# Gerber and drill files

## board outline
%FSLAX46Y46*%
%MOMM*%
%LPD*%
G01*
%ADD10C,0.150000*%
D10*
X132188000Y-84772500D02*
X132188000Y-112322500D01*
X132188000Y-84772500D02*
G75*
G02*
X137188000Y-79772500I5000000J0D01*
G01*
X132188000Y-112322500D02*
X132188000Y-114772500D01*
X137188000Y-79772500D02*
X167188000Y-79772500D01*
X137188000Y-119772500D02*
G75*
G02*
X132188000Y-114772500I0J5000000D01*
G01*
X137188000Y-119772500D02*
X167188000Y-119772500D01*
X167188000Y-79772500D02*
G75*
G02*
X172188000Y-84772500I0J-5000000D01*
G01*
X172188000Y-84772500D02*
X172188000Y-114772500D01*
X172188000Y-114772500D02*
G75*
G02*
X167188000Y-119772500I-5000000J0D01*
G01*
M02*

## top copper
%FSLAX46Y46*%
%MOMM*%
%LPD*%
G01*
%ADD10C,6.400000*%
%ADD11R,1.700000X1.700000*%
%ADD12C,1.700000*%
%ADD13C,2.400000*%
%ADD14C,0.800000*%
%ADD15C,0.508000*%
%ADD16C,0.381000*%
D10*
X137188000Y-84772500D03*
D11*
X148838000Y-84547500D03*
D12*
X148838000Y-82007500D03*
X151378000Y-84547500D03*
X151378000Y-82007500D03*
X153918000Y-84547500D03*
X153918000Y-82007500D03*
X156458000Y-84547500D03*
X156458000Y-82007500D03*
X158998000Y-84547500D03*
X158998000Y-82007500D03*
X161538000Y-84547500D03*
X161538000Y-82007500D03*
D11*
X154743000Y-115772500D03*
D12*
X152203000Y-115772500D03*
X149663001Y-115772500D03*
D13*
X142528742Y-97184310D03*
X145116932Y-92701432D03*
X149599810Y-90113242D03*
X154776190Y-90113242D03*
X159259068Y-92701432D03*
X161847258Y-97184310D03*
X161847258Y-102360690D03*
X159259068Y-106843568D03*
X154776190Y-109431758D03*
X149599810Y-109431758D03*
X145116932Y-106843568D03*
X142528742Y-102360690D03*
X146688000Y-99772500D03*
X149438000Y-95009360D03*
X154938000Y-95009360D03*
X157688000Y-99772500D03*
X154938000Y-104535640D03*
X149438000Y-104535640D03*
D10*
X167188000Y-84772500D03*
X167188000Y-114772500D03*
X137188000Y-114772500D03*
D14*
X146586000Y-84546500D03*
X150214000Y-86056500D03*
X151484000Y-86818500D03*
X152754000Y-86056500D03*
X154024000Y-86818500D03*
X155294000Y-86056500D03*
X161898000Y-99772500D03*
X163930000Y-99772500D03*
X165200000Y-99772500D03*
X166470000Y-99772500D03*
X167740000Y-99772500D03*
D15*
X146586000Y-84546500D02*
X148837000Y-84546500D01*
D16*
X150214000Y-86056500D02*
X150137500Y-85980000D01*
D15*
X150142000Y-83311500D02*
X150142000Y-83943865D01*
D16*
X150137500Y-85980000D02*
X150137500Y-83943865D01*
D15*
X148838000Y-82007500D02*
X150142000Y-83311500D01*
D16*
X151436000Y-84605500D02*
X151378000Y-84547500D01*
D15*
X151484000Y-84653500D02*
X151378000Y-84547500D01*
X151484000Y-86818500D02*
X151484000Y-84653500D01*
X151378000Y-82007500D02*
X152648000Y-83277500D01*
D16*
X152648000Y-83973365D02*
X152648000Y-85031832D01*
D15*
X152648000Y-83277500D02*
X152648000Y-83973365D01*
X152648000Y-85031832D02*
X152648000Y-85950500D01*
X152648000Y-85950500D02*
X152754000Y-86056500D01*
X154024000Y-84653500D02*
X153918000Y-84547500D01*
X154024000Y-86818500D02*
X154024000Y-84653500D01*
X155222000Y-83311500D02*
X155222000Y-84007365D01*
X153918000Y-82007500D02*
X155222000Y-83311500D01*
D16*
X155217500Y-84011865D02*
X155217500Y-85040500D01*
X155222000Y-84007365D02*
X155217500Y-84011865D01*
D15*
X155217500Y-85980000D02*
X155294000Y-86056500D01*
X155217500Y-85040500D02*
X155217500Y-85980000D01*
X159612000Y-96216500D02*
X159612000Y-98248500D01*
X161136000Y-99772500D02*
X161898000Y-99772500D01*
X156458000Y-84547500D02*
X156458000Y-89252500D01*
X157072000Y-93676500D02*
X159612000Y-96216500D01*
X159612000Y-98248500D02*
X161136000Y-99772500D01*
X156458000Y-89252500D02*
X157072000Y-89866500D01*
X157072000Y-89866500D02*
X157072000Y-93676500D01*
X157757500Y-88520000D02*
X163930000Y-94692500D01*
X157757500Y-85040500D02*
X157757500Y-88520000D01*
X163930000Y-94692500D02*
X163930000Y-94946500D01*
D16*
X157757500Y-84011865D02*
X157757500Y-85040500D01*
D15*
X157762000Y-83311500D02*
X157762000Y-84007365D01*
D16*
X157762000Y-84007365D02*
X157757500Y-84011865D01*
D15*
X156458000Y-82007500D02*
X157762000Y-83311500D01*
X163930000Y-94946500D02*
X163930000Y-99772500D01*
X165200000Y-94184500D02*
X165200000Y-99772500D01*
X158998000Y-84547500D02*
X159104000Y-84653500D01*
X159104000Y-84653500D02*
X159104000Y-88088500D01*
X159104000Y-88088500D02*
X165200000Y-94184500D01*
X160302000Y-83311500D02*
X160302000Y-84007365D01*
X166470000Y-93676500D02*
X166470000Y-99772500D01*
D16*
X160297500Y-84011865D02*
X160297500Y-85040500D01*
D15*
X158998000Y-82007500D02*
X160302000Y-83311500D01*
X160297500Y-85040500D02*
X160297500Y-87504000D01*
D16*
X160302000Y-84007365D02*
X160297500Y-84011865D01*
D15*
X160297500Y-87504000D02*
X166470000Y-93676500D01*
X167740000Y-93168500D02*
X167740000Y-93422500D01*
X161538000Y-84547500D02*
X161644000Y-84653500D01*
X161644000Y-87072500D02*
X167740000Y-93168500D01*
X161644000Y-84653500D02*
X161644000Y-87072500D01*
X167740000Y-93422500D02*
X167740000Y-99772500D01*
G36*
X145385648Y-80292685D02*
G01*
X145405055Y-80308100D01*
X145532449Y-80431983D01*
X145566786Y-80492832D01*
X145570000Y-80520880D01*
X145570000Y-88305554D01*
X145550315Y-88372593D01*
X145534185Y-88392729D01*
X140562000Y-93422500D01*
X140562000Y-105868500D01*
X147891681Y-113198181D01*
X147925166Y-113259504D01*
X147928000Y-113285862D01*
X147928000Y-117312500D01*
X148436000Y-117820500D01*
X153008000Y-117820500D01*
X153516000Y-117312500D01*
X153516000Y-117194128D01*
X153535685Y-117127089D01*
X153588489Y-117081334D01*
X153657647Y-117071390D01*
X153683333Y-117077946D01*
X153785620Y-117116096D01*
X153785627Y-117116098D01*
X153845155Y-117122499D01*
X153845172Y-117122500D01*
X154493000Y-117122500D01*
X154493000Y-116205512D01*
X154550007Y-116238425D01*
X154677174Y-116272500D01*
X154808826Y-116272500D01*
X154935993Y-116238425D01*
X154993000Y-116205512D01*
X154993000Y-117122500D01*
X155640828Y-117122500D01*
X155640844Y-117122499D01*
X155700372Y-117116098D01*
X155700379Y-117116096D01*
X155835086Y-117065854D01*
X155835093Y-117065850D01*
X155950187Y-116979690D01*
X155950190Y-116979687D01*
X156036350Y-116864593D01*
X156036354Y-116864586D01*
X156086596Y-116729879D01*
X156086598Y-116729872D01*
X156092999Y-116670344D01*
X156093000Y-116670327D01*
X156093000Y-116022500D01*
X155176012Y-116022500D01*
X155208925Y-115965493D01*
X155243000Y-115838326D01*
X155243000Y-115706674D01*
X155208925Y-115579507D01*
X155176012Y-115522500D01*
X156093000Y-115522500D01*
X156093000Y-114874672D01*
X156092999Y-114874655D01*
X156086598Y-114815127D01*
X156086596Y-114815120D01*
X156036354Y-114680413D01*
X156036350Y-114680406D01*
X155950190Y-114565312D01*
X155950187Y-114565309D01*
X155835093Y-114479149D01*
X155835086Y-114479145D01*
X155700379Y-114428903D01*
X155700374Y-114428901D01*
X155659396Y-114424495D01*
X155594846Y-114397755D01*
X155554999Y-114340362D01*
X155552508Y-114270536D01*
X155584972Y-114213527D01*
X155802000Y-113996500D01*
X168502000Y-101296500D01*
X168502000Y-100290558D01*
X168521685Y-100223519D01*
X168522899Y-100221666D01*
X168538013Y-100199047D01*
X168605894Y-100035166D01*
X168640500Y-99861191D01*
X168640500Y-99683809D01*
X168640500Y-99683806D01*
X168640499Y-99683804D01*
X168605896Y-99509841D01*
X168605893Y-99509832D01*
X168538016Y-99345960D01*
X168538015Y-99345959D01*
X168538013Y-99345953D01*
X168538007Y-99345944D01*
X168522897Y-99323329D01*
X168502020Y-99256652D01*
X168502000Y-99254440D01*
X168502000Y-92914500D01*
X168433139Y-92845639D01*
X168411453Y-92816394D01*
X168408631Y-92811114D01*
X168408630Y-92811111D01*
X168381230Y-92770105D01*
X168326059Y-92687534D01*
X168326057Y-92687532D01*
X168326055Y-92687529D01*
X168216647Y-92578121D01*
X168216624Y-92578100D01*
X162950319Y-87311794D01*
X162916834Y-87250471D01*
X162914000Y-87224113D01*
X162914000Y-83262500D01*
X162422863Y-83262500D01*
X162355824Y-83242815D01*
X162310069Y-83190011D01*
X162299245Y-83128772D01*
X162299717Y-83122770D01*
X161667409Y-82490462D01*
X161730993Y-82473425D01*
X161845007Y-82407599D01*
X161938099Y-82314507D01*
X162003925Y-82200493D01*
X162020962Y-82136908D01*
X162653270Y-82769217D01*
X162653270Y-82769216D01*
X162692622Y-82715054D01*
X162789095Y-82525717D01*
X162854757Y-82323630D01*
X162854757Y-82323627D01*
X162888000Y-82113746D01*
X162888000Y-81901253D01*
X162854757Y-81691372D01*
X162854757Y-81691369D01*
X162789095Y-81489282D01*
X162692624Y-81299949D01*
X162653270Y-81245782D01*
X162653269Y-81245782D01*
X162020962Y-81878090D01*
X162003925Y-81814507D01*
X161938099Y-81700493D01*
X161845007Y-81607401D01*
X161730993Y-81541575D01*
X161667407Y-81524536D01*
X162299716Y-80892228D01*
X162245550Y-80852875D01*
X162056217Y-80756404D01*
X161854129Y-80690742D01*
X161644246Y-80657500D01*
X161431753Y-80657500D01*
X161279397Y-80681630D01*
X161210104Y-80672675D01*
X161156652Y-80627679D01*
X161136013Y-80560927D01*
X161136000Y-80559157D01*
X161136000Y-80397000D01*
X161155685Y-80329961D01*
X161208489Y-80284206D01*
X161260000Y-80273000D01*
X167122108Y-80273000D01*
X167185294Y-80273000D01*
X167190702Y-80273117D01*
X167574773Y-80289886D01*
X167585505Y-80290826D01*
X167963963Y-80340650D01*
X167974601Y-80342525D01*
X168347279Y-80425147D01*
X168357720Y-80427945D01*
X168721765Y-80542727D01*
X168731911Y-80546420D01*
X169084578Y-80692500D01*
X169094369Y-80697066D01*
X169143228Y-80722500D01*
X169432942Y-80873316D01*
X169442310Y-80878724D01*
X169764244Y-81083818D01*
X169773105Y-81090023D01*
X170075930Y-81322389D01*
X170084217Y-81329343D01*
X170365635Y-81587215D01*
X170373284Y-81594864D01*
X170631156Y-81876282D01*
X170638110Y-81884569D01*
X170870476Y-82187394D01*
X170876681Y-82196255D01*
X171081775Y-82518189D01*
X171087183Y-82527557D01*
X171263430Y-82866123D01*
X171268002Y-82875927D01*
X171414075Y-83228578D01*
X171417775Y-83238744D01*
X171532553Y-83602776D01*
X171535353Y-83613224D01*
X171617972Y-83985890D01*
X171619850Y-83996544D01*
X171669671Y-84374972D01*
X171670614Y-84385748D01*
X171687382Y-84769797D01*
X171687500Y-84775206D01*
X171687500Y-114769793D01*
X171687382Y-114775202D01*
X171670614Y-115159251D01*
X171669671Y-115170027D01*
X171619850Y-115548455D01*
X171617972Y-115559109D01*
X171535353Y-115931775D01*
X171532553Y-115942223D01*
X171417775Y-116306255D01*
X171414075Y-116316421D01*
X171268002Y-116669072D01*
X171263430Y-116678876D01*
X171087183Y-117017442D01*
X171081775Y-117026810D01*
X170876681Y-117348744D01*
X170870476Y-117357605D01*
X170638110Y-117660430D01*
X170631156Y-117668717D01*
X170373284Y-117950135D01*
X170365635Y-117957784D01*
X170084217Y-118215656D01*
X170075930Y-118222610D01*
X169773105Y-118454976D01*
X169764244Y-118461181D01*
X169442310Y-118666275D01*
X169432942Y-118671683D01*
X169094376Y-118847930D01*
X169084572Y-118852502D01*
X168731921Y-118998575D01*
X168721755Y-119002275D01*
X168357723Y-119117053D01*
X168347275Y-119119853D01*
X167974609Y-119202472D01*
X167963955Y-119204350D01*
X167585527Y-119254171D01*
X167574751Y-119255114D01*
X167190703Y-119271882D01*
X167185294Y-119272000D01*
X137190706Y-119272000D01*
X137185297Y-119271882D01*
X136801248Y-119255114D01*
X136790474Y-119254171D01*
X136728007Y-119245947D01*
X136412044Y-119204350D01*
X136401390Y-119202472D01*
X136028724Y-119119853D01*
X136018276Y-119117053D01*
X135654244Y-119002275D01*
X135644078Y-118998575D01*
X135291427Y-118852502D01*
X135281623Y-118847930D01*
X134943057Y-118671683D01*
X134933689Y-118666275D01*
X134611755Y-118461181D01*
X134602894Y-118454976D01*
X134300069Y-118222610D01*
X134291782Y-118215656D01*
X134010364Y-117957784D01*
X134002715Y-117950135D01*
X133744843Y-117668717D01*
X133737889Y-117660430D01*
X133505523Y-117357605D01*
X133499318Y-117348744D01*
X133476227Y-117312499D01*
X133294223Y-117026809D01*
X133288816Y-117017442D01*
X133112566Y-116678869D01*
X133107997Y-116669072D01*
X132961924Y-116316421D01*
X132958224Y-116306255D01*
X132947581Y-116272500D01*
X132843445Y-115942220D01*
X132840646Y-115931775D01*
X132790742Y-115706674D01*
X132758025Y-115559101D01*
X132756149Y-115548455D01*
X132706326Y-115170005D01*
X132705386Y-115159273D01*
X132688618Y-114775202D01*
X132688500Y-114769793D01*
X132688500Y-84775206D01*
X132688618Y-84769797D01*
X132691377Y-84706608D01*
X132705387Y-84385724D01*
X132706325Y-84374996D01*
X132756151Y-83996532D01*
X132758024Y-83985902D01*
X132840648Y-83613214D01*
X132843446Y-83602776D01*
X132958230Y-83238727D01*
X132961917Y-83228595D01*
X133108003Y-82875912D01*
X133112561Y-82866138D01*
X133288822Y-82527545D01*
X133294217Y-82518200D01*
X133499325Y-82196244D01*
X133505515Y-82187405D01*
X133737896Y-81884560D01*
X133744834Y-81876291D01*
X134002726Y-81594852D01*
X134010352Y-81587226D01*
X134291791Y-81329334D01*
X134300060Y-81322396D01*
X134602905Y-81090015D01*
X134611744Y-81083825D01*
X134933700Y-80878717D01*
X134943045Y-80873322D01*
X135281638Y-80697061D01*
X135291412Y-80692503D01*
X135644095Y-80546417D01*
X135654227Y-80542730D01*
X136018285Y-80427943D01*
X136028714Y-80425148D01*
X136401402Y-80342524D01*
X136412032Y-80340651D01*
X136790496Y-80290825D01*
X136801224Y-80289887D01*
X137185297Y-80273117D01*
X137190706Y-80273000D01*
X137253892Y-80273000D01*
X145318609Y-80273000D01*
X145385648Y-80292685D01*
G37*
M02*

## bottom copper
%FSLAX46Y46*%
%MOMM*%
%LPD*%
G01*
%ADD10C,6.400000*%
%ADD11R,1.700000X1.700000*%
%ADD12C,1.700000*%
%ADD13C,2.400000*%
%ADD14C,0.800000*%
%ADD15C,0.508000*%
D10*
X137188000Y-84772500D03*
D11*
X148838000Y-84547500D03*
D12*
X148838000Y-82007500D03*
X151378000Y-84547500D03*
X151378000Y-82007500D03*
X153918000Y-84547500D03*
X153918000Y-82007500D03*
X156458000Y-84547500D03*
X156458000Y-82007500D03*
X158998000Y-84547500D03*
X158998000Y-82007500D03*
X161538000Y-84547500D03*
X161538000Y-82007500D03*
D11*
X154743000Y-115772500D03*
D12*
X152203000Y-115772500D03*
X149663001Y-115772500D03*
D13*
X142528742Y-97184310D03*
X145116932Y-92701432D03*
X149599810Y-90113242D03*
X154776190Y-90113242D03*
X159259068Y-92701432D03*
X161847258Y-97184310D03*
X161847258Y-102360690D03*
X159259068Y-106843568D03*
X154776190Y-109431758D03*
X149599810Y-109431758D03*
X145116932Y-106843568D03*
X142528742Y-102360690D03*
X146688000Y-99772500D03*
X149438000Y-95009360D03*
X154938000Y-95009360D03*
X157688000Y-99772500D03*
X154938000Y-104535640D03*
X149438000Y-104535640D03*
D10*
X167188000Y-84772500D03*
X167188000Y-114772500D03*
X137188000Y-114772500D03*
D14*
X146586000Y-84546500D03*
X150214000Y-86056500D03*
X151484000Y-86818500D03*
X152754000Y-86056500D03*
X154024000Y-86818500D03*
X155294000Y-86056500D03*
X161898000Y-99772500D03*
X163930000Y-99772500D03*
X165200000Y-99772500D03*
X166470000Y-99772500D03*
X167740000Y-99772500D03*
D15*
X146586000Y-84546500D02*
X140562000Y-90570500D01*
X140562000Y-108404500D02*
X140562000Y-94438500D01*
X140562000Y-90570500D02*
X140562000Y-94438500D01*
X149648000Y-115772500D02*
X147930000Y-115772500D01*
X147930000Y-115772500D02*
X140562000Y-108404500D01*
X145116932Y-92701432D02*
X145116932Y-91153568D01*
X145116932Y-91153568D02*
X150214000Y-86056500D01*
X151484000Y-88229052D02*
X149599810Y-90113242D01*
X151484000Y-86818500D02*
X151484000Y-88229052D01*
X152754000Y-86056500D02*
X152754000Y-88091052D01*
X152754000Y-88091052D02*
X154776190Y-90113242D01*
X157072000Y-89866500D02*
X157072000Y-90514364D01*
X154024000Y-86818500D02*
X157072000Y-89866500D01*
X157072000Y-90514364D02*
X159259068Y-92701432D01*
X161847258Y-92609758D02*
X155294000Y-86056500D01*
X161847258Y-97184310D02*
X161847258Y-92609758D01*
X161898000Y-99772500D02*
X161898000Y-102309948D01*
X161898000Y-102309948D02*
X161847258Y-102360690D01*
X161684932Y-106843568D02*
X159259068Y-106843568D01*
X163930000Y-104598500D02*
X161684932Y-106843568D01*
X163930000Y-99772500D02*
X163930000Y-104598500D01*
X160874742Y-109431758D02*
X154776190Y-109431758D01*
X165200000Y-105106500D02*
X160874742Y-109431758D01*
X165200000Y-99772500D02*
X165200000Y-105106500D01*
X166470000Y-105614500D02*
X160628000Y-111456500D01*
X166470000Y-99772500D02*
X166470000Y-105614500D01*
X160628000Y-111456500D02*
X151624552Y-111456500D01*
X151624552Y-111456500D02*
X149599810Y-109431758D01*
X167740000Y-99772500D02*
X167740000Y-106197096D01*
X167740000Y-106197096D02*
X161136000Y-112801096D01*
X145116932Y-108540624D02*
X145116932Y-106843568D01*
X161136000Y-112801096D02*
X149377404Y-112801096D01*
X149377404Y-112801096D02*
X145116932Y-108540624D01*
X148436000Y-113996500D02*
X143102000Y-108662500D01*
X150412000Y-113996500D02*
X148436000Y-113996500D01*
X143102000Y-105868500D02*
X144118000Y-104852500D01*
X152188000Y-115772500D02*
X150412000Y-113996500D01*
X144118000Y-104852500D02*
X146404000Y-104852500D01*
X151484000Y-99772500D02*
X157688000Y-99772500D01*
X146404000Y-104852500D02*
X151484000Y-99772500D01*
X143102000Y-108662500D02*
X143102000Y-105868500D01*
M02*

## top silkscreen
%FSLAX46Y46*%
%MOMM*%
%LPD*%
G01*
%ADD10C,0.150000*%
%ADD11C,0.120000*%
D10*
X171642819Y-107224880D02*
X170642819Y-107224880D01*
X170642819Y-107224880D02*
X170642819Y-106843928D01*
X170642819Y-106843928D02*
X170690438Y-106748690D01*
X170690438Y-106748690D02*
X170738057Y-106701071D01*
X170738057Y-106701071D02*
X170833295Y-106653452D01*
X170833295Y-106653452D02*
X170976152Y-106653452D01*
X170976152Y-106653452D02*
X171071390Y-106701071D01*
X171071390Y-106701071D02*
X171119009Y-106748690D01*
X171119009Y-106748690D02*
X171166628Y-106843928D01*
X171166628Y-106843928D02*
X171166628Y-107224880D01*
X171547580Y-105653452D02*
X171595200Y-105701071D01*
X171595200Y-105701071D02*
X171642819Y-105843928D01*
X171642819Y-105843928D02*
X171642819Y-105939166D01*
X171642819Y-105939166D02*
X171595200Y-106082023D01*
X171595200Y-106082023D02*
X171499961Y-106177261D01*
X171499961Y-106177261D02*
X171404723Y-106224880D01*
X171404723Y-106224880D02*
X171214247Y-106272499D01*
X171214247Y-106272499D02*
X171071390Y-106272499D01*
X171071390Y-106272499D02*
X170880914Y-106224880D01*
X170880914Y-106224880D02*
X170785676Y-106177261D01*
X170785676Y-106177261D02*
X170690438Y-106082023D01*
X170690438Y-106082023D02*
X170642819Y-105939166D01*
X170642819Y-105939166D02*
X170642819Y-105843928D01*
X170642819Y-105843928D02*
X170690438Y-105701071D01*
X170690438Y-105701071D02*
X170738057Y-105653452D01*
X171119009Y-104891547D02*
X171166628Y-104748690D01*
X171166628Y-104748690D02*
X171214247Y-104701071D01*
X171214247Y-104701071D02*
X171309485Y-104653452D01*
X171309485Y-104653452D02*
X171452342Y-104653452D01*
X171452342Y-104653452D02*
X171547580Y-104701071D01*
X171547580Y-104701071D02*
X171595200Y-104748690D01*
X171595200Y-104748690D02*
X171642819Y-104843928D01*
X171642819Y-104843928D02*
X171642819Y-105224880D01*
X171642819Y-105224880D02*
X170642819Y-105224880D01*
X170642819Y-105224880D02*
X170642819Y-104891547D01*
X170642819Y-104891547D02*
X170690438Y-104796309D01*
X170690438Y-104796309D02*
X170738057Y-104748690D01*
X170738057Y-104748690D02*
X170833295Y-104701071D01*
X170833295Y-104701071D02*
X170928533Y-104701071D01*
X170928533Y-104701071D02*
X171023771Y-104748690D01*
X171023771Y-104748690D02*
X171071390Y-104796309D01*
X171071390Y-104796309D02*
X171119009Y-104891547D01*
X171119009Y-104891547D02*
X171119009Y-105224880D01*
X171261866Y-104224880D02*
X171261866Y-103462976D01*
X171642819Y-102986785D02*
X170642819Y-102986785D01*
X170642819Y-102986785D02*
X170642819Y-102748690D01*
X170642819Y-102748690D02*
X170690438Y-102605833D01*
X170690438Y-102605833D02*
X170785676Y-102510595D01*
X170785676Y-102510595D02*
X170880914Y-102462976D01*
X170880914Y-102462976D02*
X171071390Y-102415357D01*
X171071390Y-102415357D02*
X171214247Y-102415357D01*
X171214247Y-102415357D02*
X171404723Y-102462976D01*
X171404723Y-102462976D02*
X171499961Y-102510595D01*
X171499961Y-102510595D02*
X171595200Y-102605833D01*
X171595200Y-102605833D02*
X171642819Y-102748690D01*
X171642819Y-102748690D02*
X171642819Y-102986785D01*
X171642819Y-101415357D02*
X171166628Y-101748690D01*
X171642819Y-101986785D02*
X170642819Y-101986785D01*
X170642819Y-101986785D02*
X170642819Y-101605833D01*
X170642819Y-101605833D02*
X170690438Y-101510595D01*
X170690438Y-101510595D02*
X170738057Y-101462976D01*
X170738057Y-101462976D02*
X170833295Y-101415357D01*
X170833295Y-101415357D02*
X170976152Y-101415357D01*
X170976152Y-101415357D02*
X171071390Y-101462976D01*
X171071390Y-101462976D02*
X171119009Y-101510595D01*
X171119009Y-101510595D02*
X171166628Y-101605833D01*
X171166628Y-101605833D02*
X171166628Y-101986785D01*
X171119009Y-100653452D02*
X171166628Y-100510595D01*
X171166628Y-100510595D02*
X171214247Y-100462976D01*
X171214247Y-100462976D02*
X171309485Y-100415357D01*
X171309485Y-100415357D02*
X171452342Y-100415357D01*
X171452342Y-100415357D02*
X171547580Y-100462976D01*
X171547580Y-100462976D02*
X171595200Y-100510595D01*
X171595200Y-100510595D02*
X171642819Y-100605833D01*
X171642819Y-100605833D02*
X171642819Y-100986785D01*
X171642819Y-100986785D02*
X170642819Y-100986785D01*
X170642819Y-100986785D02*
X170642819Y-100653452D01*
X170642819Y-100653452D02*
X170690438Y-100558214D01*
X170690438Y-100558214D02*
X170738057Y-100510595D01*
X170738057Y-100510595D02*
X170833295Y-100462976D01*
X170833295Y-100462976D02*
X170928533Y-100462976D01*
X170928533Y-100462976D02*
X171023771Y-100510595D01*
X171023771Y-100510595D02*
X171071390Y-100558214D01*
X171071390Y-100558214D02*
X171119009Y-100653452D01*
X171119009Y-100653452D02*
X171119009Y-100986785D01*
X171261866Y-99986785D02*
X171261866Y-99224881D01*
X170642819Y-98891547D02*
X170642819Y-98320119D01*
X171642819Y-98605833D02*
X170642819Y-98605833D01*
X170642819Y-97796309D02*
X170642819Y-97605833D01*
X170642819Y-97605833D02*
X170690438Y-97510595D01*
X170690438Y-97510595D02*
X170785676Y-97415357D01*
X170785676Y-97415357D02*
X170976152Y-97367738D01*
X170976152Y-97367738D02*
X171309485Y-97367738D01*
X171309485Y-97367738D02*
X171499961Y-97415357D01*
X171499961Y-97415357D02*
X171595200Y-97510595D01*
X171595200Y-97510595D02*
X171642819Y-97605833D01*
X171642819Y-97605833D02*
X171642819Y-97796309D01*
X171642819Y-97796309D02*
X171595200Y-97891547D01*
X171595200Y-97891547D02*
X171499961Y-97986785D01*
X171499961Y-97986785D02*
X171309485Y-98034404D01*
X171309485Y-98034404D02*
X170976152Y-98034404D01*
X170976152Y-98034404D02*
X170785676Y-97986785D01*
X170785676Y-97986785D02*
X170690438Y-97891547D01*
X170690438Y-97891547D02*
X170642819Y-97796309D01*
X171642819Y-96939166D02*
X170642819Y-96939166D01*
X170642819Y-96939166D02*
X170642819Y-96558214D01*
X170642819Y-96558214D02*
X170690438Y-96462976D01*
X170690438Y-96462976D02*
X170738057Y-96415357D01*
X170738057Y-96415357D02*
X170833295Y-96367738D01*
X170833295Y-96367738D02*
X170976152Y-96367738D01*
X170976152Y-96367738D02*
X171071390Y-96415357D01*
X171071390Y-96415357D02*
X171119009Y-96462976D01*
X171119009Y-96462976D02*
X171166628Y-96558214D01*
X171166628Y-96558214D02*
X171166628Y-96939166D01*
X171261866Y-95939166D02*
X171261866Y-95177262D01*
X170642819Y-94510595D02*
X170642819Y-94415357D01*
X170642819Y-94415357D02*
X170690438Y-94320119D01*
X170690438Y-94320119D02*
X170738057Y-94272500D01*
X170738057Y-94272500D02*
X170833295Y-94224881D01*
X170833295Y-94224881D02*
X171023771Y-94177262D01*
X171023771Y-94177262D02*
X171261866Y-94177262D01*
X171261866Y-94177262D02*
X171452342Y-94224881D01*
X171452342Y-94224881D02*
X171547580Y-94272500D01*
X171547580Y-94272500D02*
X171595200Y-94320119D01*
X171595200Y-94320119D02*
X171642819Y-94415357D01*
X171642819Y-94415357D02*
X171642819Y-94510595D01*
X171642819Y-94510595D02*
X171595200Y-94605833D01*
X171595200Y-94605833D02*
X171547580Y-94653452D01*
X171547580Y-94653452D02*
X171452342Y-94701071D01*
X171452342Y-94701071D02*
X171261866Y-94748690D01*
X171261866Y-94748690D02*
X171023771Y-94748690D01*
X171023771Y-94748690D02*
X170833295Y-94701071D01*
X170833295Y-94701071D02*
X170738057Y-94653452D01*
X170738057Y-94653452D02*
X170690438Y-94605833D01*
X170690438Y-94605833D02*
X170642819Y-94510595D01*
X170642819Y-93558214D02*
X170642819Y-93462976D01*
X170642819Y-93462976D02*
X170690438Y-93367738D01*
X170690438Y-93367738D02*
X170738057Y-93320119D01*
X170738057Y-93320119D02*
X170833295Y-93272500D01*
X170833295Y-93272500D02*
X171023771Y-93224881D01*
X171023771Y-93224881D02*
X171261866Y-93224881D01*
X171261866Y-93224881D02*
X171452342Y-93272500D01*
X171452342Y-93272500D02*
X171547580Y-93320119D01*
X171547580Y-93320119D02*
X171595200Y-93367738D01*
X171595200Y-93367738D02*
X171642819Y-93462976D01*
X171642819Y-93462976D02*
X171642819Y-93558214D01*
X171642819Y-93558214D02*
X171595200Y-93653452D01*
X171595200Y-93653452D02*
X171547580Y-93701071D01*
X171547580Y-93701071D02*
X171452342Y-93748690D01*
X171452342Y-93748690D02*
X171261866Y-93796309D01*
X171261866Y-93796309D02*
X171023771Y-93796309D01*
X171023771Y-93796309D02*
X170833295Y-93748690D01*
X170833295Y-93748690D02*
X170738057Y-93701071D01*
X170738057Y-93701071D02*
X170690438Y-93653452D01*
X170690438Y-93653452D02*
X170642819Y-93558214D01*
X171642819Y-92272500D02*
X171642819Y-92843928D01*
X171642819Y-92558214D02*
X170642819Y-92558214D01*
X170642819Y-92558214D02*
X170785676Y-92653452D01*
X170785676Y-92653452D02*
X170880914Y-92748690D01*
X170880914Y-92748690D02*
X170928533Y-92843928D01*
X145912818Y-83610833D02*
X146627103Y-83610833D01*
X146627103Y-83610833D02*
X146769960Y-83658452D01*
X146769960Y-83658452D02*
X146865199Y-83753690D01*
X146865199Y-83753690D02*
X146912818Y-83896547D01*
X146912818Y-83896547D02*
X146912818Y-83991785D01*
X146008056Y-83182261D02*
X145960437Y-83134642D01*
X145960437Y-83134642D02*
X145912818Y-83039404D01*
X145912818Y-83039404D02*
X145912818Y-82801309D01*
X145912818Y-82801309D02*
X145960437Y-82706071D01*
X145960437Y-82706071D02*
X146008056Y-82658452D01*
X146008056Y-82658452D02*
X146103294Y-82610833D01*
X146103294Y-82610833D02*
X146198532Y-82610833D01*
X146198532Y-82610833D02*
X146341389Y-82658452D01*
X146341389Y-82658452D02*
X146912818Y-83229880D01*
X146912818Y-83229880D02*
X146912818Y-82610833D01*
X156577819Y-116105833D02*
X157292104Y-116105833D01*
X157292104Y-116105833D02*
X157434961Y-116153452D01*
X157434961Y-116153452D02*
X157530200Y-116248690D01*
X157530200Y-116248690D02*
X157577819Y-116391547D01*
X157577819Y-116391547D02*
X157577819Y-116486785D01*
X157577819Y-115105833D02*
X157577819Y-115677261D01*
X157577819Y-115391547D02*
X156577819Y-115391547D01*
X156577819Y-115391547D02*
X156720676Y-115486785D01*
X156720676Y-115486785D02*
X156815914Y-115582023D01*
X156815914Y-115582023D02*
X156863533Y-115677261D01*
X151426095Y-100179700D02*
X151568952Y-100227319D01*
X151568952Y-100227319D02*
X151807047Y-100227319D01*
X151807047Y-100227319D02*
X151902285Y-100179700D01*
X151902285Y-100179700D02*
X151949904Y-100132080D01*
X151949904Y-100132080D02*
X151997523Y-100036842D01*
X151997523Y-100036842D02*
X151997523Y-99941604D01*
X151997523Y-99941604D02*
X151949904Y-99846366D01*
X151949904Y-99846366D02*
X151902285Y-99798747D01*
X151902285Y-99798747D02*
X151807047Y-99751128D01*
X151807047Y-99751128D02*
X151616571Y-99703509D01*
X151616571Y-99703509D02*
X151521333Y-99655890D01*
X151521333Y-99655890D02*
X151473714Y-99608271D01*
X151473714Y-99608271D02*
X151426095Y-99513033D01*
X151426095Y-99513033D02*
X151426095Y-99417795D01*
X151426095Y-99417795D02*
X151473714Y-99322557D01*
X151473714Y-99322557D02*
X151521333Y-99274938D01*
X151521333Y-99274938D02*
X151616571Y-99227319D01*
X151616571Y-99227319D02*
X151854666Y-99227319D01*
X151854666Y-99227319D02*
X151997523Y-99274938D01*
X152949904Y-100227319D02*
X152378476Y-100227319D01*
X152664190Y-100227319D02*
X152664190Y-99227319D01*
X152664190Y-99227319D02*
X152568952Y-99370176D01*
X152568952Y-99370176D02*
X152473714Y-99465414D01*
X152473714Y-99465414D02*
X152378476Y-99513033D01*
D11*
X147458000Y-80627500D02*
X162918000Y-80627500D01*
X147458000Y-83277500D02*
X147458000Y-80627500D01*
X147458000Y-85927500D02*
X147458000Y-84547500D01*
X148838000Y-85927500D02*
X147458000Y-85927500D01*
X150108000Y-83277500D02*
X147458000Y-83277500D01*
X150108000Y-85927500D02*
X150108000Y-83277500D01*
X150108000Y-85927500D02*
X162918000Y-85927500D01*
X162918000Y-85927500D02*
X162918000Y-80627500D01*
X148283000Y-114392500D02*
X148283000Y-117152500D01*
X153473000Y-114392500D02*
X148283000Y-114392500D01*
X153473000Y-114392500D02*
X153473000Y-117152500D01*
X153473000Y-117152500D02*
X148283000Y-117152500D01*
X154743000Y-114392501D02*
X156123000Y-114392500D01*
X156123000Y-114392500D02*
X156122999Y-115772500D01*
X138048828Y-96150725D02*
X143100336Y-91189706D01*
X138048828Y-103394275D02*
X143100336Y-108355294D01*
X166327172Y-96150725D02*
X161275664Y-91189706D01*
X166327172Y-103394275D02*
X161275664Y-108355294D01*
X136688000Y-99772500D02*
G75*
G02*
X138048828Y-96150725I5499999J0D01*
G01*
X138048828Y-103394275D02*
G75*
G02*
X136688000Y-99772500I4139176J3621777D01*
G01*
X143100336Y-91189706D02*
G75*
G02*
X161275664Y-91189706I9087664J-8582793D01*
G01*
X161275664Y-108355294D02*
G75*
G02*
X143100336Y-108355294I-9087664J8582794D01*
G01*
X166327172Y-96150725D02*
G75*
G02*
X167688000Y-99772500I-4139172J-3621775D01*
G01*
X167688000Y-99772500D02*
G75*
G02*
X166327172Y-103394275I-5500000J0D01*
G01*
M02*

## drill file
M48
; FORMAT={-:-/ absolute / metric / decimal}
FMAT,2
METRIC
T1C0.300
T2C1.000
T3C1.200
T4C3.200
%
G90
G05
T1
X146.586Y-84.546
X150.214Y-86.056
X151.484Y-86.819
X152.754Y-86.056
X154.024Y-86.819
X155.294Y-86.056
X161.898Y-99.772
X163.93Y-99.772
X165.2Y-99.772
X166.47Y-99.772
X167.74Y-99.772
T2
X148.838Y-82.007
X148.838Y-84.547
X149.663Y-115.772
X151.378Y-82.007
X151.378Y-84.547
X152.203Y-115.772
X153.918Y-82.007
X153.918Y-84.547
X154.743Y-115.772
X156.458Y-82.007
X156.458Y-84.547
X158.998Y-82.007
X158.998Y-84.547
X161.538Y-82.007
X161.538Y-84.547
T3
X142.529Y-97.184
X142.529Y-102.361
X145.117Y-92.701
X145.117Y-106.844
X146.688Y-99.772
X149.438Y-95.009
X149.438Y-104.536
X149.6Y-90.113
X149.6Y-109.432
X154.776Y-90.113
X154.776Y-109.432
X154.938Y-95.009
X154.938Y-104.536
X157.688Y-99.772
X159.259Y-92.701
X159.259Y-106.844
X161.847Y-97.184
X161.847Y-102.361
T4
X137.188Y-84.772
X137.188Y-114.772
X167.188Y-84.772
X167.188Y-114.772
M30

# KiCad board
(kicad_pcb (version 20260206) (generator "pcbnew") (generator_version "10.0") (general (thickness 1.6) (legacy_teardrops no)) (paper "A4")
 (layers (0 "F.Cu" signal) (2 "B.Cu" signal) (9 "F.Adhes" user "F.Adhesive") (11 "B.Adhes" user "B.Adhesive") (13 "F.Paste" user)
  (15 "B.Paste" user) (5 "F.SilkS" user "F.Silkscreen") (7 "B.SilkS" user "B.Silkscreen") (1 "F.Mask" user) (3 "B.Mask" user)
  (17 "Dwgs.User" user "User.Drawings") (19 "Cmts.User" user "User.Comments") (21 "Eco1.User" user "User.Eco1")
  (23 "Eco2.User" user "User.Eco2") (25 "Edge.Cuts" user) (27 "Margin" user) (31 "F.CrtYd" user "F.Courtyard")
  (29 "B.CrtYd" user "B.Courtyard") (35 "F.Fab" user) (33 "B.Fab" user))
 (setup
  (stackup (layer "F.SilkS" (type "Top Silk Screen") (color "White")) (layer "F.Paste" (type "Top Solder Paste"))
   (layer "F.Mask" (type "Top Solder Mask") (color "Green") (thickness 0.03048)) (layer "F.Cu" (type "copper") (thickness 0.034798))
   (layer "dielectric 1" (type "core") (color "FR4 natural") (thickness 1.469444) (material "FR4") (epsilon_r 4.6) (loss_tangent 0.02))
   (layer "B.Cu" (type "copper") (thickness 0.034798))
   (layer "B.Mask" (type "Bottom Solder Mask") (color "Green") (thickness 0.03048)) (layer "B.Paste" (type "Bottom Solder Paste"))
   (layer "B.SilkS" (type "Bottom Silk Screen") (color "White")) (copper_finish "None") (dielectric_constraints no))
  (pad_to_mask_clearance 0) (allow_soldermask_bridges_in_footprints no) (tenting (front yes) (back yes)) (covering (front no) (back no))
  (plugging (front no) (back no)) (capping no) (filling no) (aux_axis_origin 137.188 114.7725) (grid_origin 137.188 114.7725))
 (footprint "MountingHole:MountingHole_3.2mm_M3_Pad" (layer "F.Cu") (at 137.188 84.7725)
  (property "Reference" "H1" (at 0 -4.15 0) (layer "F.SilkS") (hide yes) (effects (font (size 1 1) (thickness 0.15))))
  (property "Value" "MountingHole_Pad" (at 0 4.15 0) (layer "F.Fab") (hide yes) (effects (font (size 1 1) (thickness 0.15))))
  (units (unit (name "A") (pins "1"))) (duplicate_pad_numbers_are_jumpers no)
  (pad "1" thru_hole circle (at 0 0) (size 6.4 6.4) (drill 3.2) (layers "*.Cu" "*.Mask") (remove_unused_layers no) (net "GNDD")
   (zone_connect 2)))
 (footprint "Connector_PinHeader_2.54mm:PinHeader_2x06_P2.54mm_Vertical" (layer "F.Cu") (at 148.838 84.5475 90)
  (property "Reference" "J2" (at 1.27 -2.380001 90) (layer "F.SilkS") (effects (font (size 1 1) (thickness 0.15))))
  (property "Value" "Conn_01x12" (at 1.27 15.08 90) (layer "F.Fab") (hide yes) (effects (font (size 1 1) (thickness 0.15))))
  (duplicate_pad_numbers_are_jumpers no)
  (fp_line (start 3.92 -1.38) (end 3.92 14.08) (stroke (width 0.12) (type solid)) (layer "F.SilkS"))
  (fp_line (start 1.27 -1.38) (end 3.92 -1.38) (stroke (width 0.12) (type solid)) (layer "F.SilkS"))
  (fp_line (start -1.38 -1.38) (end 0 -1.38) (stroke (width 0.12) (type solid)) (layer "F.SilkS"))
  (fp_line (start -1.38 0) (end -1.38 -1.38) (stroke (width 0.12) (type solid)) (layer "F.SilkS"))
  (fp_line (start 1.27 1.27) (end 1.27 -1.38) (stroke (width 0.12) (type solid)) (layer "F.SilkS"))
  (fp_line (start -1.38 1.27) (end 1.27 1.27) (stroke (width 0.12) (type solid)) (layer "F.SilkS"))
  (fp_line (start -1.38 1.27) (end -1.38 14.08) (stroke (width 0.12) (type solid)) (layer "F.SilkS"))
  (fp_line (start -1.38 14.08) (end 3.92 14.08) (stroke (width 0.12) (type solid)) (layer "F.SilkS"))
  (pad "1" thru_hole rect (at 0 0 90) (size 1.7 1.7) (drill 1) (layers "*.Cu" "*.Mask") (remove_unused_layers no) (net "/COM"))
  (pad "2" thru_hole circle (at 2.54 0 90) (size 1.7 1.7) (drill 1) (layers "*.Cu" "*.Mask") (remove_unused_layers no) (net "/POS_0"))
  (pad "3" thru_hole circle (at 0 2.54 90) (size 1.7 1.7) (drill 1) (layers "*.Cu" "*.Mask") (remove_unused_layers no) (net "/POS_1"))
  (pad "4" thru_hole circle (at 2.54 2.54 90) (size 1.7 1.7) (drill 1) (layers "*.Cu" "*.Mask") (remove_unused_layers no) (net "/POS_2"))
  (pad "5" thru_hole circle (at 0 5.08 90) (size 1.7 1.7) (drill 1) (layers "*.Cu" "*.Mask") (remove_unused_layers no) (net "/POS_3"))
  (pad "6" thru_hole circle (at 2.54 5.08 90) (size 1.7 1.7) (drill 1) (layers "*.Cu" "*.Mask") (remove_unused_layers no) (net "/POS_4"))
  (pad "7" thru_hole circle (at 0 7.62 90) (size 1.7 1.7) (drill 1) (layers "*.Cu" "*.Mask") (remove_unused_layers no) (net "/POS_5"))
  (pad "8" thru_hole circle (at 2.54 7.62 90) (size 1.7 1.7) (drill 1) (layers "*.Cu" "*.Mask") (remove_unused_layers no) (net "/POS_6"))
  (pad "9" thru_hole circle (at 0 10.16 90) (size 1.7 1.7) (drill 1) (layers "*.Cu" "*.Mask") (remove_unused_layers no) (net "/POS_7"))
  (pad "10" thru_hole circle (at 2.54 10.16 90) (size 1.7 1.7) (drill 1) (layers "*.Cu" "*.Mask") (remove_unused_layers no) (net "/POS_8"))
  (pad "11" thru_hole circle (at 0 12.7 90) (size 1.7 1.7) (drill 1) (layers "*.Cu" "*.Mask") (remove_unused_layers no) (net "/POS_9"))
  (pad "12" thru_hole circle (at 2.54 12.7 90) (size 1.7 1.7) (drill 1) (layers "*.Cu" "*.Mask") (remove_unused_layers no) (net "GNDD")))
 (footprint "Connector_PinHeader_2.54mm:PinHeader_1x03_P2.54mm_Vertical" (layer "F.Cu") (at 154.743 115.7725 -90)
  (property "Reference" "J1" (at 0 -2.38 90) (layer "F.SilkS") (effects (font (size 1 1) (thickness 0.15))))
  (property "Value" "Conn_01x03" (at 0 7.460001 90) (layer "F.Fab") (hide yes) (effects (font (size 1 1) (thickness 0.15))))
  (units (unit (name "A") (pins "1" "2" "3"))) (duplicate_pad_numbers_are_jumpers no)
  (fp_line (start -1.38 6.46) (end 1.38 6.46) (stroke (width 0.12) (type solid)) (layer "F.SilkS"))
  (fp_line (start -1.38 1.27) (end -1.38 6.46) (stroke (width 0.12) (type solid)) (layer "F.SilkS"))
  (fp_line (start -1.38 1.27) (end 1.38 1.27) (stroke (width 0.12) (type solid)) (layer "F.SilkS"))
  (fp_line (start 1.38 1.27) (end 1.38 6.46) (stroke (width 0.12) (type solid)) (layer "F.SilkS"))
  (fp_line (start -1.379999 0) (end -1.38 -1.38) (stroke (width 0.12) (type solid)) (layer "F.SilkS"))
  (fp_line (start -1.38 -1.38) (end 0 -1.379999) (stroke (width 0.12) (type solid)) (layer "F.SilkS"))
  (pad "1" thru_hole rect (at 0 0 270) (size 1.7 1.7) (drill 1) (layers "*.Cu" "*.Mask") (remove_unused_layers no) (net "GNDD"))
  (pad "2" thru_hole circle (at 0 2.54 270) (size 1.7 1.7) (drill 1) (layers "*.Cu" "*.Mask") (remove_unused_layers no) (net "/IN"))
  (pad "3" thru_hole circle (at 0 5.079999 270) (size 1.7 1.7) (drill 1) (layers "*.Cu" "*.Mask") (remove_unused_layers no) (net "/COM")))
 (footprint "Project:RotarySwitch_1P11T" (layer "F.Cu") (at 152.188 99.7725 -90)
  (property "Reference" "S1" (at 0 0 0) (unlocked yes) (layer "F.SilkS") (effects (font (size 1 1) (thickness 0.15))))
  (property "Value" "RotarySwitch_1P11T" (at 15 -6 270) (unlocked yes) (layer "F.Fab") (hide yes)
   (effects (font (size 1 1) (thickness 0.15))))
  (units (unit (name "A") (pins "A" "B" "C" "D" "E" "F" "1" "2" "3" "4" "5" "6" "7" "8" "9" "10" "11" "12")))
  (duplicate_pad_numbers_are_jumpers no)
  (fp_line (start -3.621775 14.139172) (end -8.582794 9.087664) (stroke (width 0.12) (type default)) (layer "F.SilkS"))
  (fp_line (start 3.621775 14.139172) (end 8.582794 9.087664) (stroke (width 0.12) (type default)) (layer "F.SilkS"))
  (fp_line (start -3.621775 -14.139172) (end -8.582794 -9.087664) (stroke (width 0.12) (type default)) (layer "F.SilkS"))
  (fp_line (start 3.621775 -14.139172) (end 8.582794 -9.087664) (stroke (width 0.12) (type default)) (layer "F.SilkS"))
  (fp_arc (start 0 15.5) (mid -1.934497 15.148565) (end -3.621775 14.139172) (stroke (width 0.12) (type default)) (layer "F.SilkS"))
  (fp_arc (start 3.621775 14.139172) (mid 1.934496 15.148565) (end 0 15.5) (stroke (width 0.12) (type default)) (layer "F.SilkS"))
  (fp_arc (start -8.582794 9.087664) (mid -12.5 0) (end -8.582794 -9.087664) (stroke (width 0.12) (type default)) (layer "F.SilkS"))
  (fp_arc (start 8.582794 -9.087664) (mid 12.5 0) (end 8.582794 9.087664) (stroke (width 0.12) (type default)) (layer "F.SilkS"))
  (fp_arc (start -3.621775 -14.139172) (mid -1.934496 -15.148565) (end 0 -15.5) (stroke (width 0.12) (type default)) (layer "F.SilkS"))
  (fp_arc (start 0 -15.5) (mid 1.934497 -15.148565) (end 3.621775 -14.139172) (stroke (width 0.12) (type default)) (layer "F.SilkS"))
  (pad "1" thru_hole circle (at -2.58819 9.659258 270) (size 2.4 2.4) (drill 1.2) (layers "*.Cu" "*.Mask") (remove_unused_layers no)
   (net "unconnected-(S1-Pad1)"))
  (pad "2" thru_hole circle (at -7.071068 7.071068 270) (size 2.4 2.4) (drill 1.2) (layers "*.Cu" "*.Mask") (remove_unused_layers no)
   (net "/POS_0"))
  (pad "3" thru_hole circle (at -9.659258 2.58819 270) (size 2.4 2.4) (drill 1.2) (layers "*.Cu" "*.Mask") (remove_unused_layers no)
   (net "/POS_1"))
  (pad "4" thru_hole circle (at -9.659258 -2.58819 270) (size 2.4 2.4) (drill 1.2) (layers "*.Cu" "*.Mask") (remove_unused_layers no)
   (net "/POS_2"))
  (pad "5" thru_hole circle (at -7.071068 -7.071068 270) (size 2.4 2.4) (drill 1.2) (layers "*.Cu" "*.Mask") (remove_unused_layers no)
   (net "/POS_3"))
  (pad "6" thru_hole circle (at -2.58819 -9.659258 270) (size 2.4 2.4) (drill 1.2) (layers "*.Cu" "*.Mask") (remove_unused_layers no)
   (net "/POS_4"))
  (pad "7" thru_hole circle (at 2.58819 -9.659258 270) (size 2.4 2.4) (drill 1.2) (layers "*.Cu" "*.Mask") (remove_unused_layers no)
   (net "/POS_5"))
  (pad "8" thru_hole circle (at 7.071068 -7.071068 270) (size 2.4 2.4) (drill 1.2) (layers "*.Cu" "*.Mask") (remove_unused_layers no)
   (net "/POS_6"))
  (pad "9" thru_hole circle (at 9.659258 -2.58819 270) (size 2.4 2.4) (drill 1.2) (layers "*.Cu" "*.Mask") (remove_unused_layers no)
   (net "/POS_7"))
  (pad "10" thru_hole circle (at 9.659258 2.58819 270) (size 2.4 2.4) (drill 1.2) (layers "*.Cu" "*.Mask") (remove_unused_layers no)
   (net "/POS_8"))
  (pad "11" thru_hole circle (at 7.071068 7.071068 270) (size 2.4 2.4) (drill 1.2) (layers "*.Cu" "*.Mask") (remove_unused_layers no)
   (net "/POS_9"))
  (pad "12" thru_hole circle (at 2.58819 9.659258 270) (size 2.4 2.4) (drill 1.2) (layers "*.Cu" "*.Mask") (remove_unused_layers no)
   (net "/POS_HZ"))
  (pad "A" thru_hole circle (at 0 5.5 270) (size 2.4 2.4) (drill 1.2) (layers "*.Cu" "*.Mask") (remove_unused_layers no)
   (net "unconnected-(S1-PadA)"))
  (pad "B" thru_hole circle (at -4.76314 2.75 270) (size 2.4 2.4) (drill 1.2) (layers "*.Cu" "*.Mask") (remove_unused_layers no)
   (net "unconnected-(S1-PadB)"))
  (pad "C" thru_hole circle (at -4.76314 -2.75 270) (size 2.4 2.4) (drill 1.2) (layers "*.Cu" "*.Mask") (remove_unused_layers no)
   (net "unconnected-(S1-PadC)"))
  (pad "D" thru_hole circle (at 0 -5.5 270) (size 2.4 2.4) (drill 1.2) (layers "*.Cu" "*.Mask") (remove_unused_layers no) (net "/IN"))
  (pad "E" thru_hole circle (at 4.76314 -2.75 270) (size 2.4 2.4) (drill 1.2) (layers "*.Cu" "*.Mask") (remove_unused_layers no)
   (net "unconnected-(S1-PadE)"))
  (pad "F" thru_hole circle (at 4.76314 2.75 270) (size 2.4 2.4) (drill 1.2) (layers "*.Cu" "*.Mask") (remove_unused_layers no)
   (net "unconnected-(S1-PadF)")))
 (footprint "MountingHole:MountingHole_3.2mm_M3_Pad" (layer "F.Cu") (at 167.188 84.7725)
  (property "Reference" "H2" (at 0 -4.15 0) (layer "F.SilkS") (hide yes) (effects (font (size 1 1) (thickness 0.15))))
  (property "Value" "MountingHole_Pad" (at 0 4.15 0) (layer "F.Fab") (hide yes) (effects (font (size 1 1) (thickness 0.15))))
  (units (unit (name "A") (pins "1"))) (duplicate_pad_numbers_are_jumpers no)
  (pad "1" thru_hole circle (at 0 0) (size 6.4 6.4) (drill 3.2) (layers "*.Cu" "*.Mask") (remove_unused_layers no) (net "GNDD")
   (zone_connect 2)))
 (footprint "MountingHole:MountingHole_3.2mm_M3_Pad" (layer "F.Cu") (at 167.188 114.7725)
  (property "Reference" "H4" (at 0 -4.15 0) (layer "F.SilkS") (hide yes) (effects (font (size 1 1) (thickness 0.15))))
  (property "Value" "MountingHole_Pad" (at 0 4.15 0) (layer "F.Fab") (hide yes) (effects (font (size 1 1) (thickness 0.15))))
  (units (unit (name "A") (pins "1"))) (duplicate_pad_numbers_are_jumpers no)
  (pad "1" thru_hole circle (at 0 0) (size 6.4 6.4) (drill 3.2) (layers "*.Cu" "*.Mask") (remove_unused_layers no) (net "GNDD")
   (zone_connect 2)))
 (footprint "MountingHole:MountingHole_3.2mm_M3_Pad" (layer "F.Cu") (at 137.188 114.7725)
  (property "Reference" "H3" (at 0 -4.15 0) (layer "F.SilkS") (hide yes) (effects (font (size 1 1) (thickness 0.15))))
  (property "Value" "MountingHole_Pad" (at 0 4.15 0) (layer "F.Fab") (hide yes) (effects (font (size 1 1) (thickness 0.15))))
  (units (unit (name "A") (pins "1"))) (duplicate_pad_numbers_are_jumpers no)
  (pad "1" thru_hole circle (at 0 0) (size 6.4 6.4) (drill 3.2) (layers "*.Cu" "*.Mask") (remove_unused_layers no) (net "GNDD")
   (zone_connect 2)))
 (gr_line (start 132.188 84.7725) (end 132.188 112.3225) (stroke (width 0.15) (type default)) (layer "Edge.Cuts"))
 (gr_arc (start 132.188 84.7725) (mid 133.652466 81.236966) (end 137.188 79.7725) (stroke (width 0.15) (type default)) (layer "Edge.Cuts"))
 (gr_line (start 132.188 112.3225) (end 132.188 114.7725) (stroke (width 0.15) (type default)) (layer "Edge.Cuts"))
 (gr_line (start 137.188 79.7725) (end 167.188 79.7725) (stroke (width 0.15) (type default)) (layer "Edge.Cuts"))
 (gr_arc (start 137.188 119.7725) (mid 133.652466 118.308034) (end 132.188 114.7725) (stroke (width 0.15) (type default))
  (layer "Edge.Cuts"))
 (gr_line (start 137.188 119.7725) (end 167.188 119.7725) (stroke (width 0.15) (type default)) (layer "Edge.Cuts"))
 (gr_arc (start 167.188 79.7725) (mid 170.723534 81.236966) (end 172.188 84.7725) (stroke (width 0.15) (type default)) (layer "Edge.Cuts"))
 (gr_line (start 172.188 84.7725) (end 172.188 114.7725) (stroke (width 0.15) (type default)) (layer "Edge.Cuts"))
 (gr_arc (start 172.188 114.7725) (mid 170.723534 118.308034) (end 167.188 119.7725) (stroke (width 0.15) (type default))
  (layer "Edge.Cuts"))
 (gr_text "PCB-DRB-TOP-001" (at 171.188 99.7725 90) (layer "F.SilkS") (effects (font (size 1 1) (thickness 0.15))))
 (segment (start 146.586 84.5465) (end 148.837 84.5465) (width 0.508) (layer "F.Cu") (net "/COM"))
 (via (at 146.586 84.5465) (size 0.8) (drill 0.3) (layers "F.Cu" "B.Cu") (capping no) (covering (front no) (back no))
  (plugging (front no) (back no)) (filling no) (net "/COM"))
 (segment (start 146.586 84.5465) (end 140.562 90.5705) (width 0.508) (layer "B.Cu") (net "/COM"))
 (segment (start 140.562 108.4045) (end 140.562 94.4385) (width 0.508) (layer "B.Cu") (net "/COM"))
 (segment (start 140.562 90.5705) (end 140.562 94.4385) (width 0.508) (layer "B.Cu") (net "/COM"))
 (segment (start 149.648 115.7725) (end 147.93 115.7725) (width 0.508) (layer "B.Cu") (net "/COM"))
 (segment (start 147.93 115.7725) (end 140.562 108.4045) (width 0.508) (layer "B.Cu") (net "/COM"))
 (segment (start 150.214 86.0565) (end 150.1375 85.98) (width 0.381) (layer "F.Cu") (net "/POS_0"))
 (segment (start 150.142 83.3115) (end 150.142 83.943865) (width 0.508) (layer "F.Cu") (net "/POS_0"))
 (segment (start 150.1375 85.98) (end 150.1375 83.943865) (width 0.381) (layer "F.Cu") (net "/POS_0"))
 (segment (start 148.838 82.0075) (end 150.142 83.3115) (width 0.508) (layer "F.Cu") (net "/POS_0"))
 (via (at 150.214 86.0565) (size 0.8) (drill 0.3) (layers "F.Cu" "B.Cu") (capping no) (covering (front no) (back no))
  (plugging (front no) (back no)) (filling no) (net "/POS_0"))
 (segment (start 145.116932 92.701432) (end 145.116932 91.153568) (width 0.508) (layer "B.Cu") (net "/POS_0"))
 (segment (start 145.116932 91.153568) (end 150.214 86.0565) (width 0.508) (layer "B.Cu") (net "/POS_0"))
 (segment (start 151.436 84.6055) (end 151.378 84.5475) (width 0.381) (layer "F.Cu") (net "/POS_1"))
 (segment (start 151.484 84.6535) (end 151.378 84.5475) (width 0.508) (layer "F.Cu") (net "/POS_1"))
 (segment (start 151.484 86.8185) (end 151.484 84.6535) (width 0.508) (layer "F.Cu") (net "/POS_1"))
 (via (at 151.484 86.8185) (size 0.8) (drill 0.3) (layers "F.Cu" "B.Cu") (capping no) (covering (front no) (back no))
  (plugging (front no) (back no)) (filling no) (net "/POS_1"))
 (segment (start 151.484 88.229052) (end 149.59981 90.113242) (width 0.508) (layer "B.Cu") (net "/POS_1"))
 (segment (start 151.484 86.8185) (end 151.484 88.229052) (width 0.508) (layer "B.Cu") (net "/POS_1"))
 (segment (start 151.378 82.0075) (end 152.648 83.2775) (width 0.508) (layer "F.Cu") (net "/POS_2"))
 (segment (start 152.648 83.973365) (end 152.648 85.031832) (width 0.381) (layer "F.Cu") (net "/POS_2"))
 (segment (start 152.648 83.2775) (end 152.648 83.973365) (width 0.508) (layer "F.Cu") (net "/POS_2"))
 (segment (start 152.648 85.031832) (end 152.648 85.9505) (width 0.508) (layer "F.Cu") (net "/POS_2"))
 (segment (start 152.648 85.9505) (end 152.754 86.0565) (width 0.508) (layer "F.Cu") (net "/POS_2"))
 (via (at 152.754 86.0565) (size 0.8) (drill 0.3) (layers "F.Cu" "B.Cu") (capping no) (covering (front no) (back no))
  (plugging (front no) (back no)) (filling no) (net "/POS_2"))
 (segment (start 152.754 86.0565) (end 152.754 88.091052) (width 0.508) (layer "B.Cu") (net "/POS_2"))
 (segment (start 152.754 88.091052) (end 154.77619 90.113242) (width 0.508) (layer "B.Cu") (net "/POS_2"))
 (segment (start 154.024 84.6535) (end 153.918 84.5475) (width 0.508) (layer "F.Cu") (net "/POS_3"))
 (segment (start 154.024 86.8185) (end 154.024 84.6535) (width 0.508) (layer "F.Cu") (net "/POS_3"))
 (via (at 154.024 86.8185) (size 0.8) (drill 0.3) (layers "F.Cu" "B.Cu") (capping no) (covering (front no) (back no))
  (plugging (front no) (back no)) (filling no) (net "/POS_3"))
 (segment (start 157.072 89.8665) (end 157.072 90.514364) (width 0.508) (layer "B.Cu") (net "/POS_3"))
 (segment (start 154.024 86.8185) (end 157.072 89.8665) (width 0.508) (layer "B.Cu") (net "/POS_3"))
 (segment (start 157.072 90.514364) (end 159.259068 92.701432) (width 0.508) (layer "B.Cu") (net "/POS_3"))
 (segment (start 155.222 83.3115) (end 155.222 84.007365) (width 0.508) (layer "F.Cu") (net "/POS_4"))
 (segment (start 153.918 82.0075) (end 155.222 83.3115) (width 0.508) (layer "F.Cu") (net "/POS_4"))
 (segment (start 155.2175 84.011865) (end 155.2175 85.0405) (width 0.381) (layer "F.Cu") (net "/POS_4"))
 (segment (start 155.222 84.007365) (end 155.2175 84.011865) (width 0.381) (layer "F.Cu") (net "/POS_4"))
 (segment (start 155.2175 85.98) (end 155.294 86.0565) (width 0.508) (layer "F.Cu") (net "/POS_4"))
 (segment (start 155.2175 85.0405) (end 155.2175 85.98) (width 0.508) (layer "F.Cu") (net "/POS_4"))
 (via (at 155.294 86.0565) (size 0.8) (drill 0.3) (layers "F.Cu" "B.Cu") (capping no) (covering (front no) (back no))
  (plugging (front no) (back no)) (filling no) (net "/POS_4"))
 (segment (start 161.847258 92.609758) (end 155.294 86.0565) (width 0.508) (layer "B.Cu") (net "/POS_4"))
 (segment (start 161.847258 97.18431) (end 161.847258 92.609758) (width 0.508) (layer "B.Cu") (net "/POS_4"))
 (segment (start 159.612 96.2165) (end 159.612 98.2485) (width 0.508) (layer "F.Cu") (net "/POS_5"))
 (segment (start 161.136 99.7725) (end 161.898 99.7725) (width 0.508) (layer "F.Cu") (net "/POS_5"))
 (segment (start 156.458 84.5475) (end 156.458 89.2525) (width 0.508) (layer "F.Cu") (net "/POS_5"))
 (segment (start 157.072 93.6765) (end 159.612 96.2165) (width 0.508) (layer "F.Cu") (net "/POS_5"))
 (segment (start 159.612 98.2485) (end 161.136 99.7725) (width 0.508) (layer "F.Cu") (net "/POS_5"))
 (segment (start 156.458 89.2525) (end 157.072 89.8665) (width 0.508) (layer "F.Cu") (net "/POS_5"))
 (segment (start 157.072 89.8665) (end 157.072 93.6765) (width 0.508) (layer "F.Cu") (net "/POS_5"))
 (via (at 161.898 99.7725) (size 0.8) (drill 0.3) (layers "F.Cu" "B.Cu") (capping no) (covering (front no) (back no))
  (plugging (front no) (back no)) (filling no) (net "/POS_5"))
 (segment (start 161.898 99.7725) (end 161.898 102.309948) (width 0.508) (layer "B.Cu") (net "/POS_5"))
 (segment (start 161.898 102.309948) (end 161.847258 102.36069) (width 0.508) (layer "B.Cu") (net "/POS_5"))
 (segment (start 157.7575 88.52) (end 163.93 94.6925) (width 0.508) (layer "F.Cu") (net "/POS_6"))
 (segment (start 157.7575 85.0405) (end 157.7575 88.52) (width 0.508) (layer "F.Cu") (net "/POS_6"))
 (segment (start 163.93 94.6925) (end 163.93 94.9465) (width 0.508) (layer "F.Cu") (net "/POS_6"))
 (segment (start 157.7575 84.011865) (end 157.7575 85.0405) (width 0.381) (layer "F.Cu") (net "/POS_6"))
 (segment (start 157.762 83.3115) (end 157.762 84.007365) (width 0.508) (layer "F.Cu") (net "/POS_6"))
 (segment (start 157.762 84.007365) (end 157.7575 84.011865) (width 0.381) (layer "F.Cu") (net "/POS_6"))
 (segment (start 156.458 82.0075) (end 157.762 83.3115) (width 0.508) (layer "F.Cu") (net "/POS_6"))
 (segment (start 163.93 94.9465) (end 163.93 99.7725) (width 0.508) (layer "F.Cu") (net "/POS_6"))
 (via (at 163.93 99.7725) (size 0.8) (drill 0.3) (layers "F.Cu" "B.Cu") (capping no) (covering (front no) (back no))
  (plugging (front no) (back no)) (filling no) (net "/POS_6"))
 (segment (start 161.684932 106.843568) (end 159.259068 106.843568) (width 0.508) (layer "B.Cu") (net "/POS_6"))
 (segment (start 163.93 104.5985) (end 161.684932 106.843568) (width 0.508) (layer "B.Cu") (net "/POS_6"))
 (segment (start 163.93 99.7725) (end 163.93 104.5985) (width 0.508) (layer "B.Cu") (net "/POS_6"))
 (segment (start 165.2 94.1845) (end 165.2 99.7725) (width 0.508) (layer "F.Cu") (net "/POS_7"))
 (segment (start 158.998 84.5475) (end 159.104 84.6535) (width 0.508) (layer "F.Cu") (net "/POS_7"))
 (segment (start 159.104 84.6535) (end 159.104 88.0885) (width 0.508) (layer "F.Cu") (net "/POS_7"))
 (segment (start 159.104 88.0885) (end 165.2 94.1845) (width 0.508) (layer "F.Cu") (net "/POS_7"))
 (via (at 165.2 99.7725) (size 0.8) (drill 0.3) (layers "F.Cu" "B.Cu") (capping no) (covering (front no) (back no))
  (plugging (front no) (back no)) (filling no) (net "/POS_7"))
 (segment (start 160.874742 109.431758) (end 154.77619 109.431758) (width 0.508) (layer "B.Cu") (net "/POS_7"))
 (segment (start 165.2 105.1065) (end 160.874742 109.431758) (width 0.508) (layer "B.Cu") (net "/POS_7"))
 (segment (start 165.2 99.7725) (end 165.2 105.1065) (width 0.508) (layer "B.Cu") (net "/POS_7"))
 (segment (start 160.302 83.3115) (end 160.302 84.007365) (width 0.508) (layer "F.Cu") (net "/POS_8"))
 (segment (start 166.47 93.6765) (end 166.47 99.7725) (width 0.508) (layer "F.Cu") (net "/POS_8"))
 (segment (start 160.2975 84.011865) (end 160.2975 85.0405) (width 0.381) (layer "F.Cu") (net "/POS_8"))
 (segment (start 158.998 82.0075) (end 160.302 83.3115) (width 0.508) (layer "F.Cu") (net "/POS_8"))
 (segment (start 160.2975 85.0405) (end 160.2975 87.504) (width 0.508) (layer "F.Cu") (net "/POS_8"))
 (segment (start 160.302 84.007365) (end 160.2975 84.011865) (width 0.381) (layer "F.Cu") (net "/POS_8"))
 (segment (start 160.2975 87.504) (end 166.47 93.6765) (width 0.508) (layer "F.Cu") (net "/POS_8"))
 (via (at 166.47 99.7725) (size 0.8) (drill 0.3) (layers "F.Cu" "B.Cu") (capping no) (covering (front no) (back no))
  (plugging (front no) (back no)) (filling no) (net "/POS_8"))
 (segment (start 166.47 105.6145) (end 160.628 111.4565) (width 0.508) (layer "B.Cu") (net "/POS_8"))
 (segment (start 166.47 99.7725) (end 166.47 105.6145) (width 0.508) (layer "B.Cu") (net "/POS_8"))
 (segment (start 160.628 111.4565) (end 151.624552 111.4565) (width 0.508) (layer "B.Cu") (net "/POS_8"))
 (segment (start 151.624552 111.4565) (end 149.59981 109.431758) (width 0.508) (layer "B.Cu") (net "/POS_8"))
 (segment (start 167.74 93.1685) (end 167.74 93.4225) (width 0.508) (layer "F.Cu") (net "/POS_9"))
 (segment (start 161.538 84.5475) (end 161.644 84.6535) (width 0.508) (layer "F.Cu") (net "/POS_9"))
 (segment (start 161.644 87.0725) (end 167.74 93.1685) (width 0.508) (layer "F.Cu") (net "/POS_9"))
 (segment (start 161.644 84.6535) (end 161.644 87.0725) (width 0.508) (layer "F.Cu") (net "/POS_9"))
 (segment (start 167.74 93.4225) (end 167.74 99.7725) (width 0.508) (layer "F.Cu") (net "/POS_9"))
 (via (at 167.74 99.7725) (size 0.8) (drill 0.3) (layers "F.Cu" "B.Cu") (capping no) (covering (front no) (back no))
  (plugging (front no) (back no)) (filling no) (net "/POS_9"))
 (segment (start 167.74 99.7725) (end 167.74 106.197096) (width 0.508) (layer "B.Cu") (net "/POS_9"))
 (segment (start 167.74 106.197096) (end 161.136 112.801096) (width 0.508) (layer "B.Cu") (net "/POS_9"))
 (segment (start 145.116932 108.540624) (end 145.116932 106.843568) (width 0.508) (layer "B.Cu") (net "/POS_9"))
 (segment (start 161.136 112.801096) (end 149.377404 112.801096) (width 0.508) (layer "B.Cu") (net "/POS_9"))
 (segment (start 149.377404 112.801096) (end 145.116932 108.540624) (width 0.508) (layer "B.Cu") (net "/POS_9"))
 (segment (start 148.436 113.9965) (end 143.102 108.6625) (width 0.508) (layer "B.Cu") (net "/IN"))
 (segment (start 150.412 113.9965) (end 148.436 113.9965) (width 0.508) (layer "B.Cu") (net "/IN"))
 (segment (start 143.102 105.8685) (end 144.118 104.8525) (width 0.508) (layer "B.Cu") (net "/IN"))
 (segment (start 152.188 115.7725) (end 150.412 113.9965) (width 0.508) (layer "B.Cu") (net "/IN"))
 (segment (start 144.118 104.8525) (end 146.404 104.8525) (width 0.508) (layer "B.Cu") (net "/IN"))
 (segment (start 151.484 99.7725) (end 157.688 99.7725) (width 0.508) (layer "B.Cu") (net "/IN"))
 (segment (start 146.404 104.8525) (end 151.484 99.7725) (width 0.508) (layer "B.Cu") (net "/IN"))
 (segment (start 143.102 108.6625) (end 143.102 105.8685) (width 0.508) (layer "B.Cu") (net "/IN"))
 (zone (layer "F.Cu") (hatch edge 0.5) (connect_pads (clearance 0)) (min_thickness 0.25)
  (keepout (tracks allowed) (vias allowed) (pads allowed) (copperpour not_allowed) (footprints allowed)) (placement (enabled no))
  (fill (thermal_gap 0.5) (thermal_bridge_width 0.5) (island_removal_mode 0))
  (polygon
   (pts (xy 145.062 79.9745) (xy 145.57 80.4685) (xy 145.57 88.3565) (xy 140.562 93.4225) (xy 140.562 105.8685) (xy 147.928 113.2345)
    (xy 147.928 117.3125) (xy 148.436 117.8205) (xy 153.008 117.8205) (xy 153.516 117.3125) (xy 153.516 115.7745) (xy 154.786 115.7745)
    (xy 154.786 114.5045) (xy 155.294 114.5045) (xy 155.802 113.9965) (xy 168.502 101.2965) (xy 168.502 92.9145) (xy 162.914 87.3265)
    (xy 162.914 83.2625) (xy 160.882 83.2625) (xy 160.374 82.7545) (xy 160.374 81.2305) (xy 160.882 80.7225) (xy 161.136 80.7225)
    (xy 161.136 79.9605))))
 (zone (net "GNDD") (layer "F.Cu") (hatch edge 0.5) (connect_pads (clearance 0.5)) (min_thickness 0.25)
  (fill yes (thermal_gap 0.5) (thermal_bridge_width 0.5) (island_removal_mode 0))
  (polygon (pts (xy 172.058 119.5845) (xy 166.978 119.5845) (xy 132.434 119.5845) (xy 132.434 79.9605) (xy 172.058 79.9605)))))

